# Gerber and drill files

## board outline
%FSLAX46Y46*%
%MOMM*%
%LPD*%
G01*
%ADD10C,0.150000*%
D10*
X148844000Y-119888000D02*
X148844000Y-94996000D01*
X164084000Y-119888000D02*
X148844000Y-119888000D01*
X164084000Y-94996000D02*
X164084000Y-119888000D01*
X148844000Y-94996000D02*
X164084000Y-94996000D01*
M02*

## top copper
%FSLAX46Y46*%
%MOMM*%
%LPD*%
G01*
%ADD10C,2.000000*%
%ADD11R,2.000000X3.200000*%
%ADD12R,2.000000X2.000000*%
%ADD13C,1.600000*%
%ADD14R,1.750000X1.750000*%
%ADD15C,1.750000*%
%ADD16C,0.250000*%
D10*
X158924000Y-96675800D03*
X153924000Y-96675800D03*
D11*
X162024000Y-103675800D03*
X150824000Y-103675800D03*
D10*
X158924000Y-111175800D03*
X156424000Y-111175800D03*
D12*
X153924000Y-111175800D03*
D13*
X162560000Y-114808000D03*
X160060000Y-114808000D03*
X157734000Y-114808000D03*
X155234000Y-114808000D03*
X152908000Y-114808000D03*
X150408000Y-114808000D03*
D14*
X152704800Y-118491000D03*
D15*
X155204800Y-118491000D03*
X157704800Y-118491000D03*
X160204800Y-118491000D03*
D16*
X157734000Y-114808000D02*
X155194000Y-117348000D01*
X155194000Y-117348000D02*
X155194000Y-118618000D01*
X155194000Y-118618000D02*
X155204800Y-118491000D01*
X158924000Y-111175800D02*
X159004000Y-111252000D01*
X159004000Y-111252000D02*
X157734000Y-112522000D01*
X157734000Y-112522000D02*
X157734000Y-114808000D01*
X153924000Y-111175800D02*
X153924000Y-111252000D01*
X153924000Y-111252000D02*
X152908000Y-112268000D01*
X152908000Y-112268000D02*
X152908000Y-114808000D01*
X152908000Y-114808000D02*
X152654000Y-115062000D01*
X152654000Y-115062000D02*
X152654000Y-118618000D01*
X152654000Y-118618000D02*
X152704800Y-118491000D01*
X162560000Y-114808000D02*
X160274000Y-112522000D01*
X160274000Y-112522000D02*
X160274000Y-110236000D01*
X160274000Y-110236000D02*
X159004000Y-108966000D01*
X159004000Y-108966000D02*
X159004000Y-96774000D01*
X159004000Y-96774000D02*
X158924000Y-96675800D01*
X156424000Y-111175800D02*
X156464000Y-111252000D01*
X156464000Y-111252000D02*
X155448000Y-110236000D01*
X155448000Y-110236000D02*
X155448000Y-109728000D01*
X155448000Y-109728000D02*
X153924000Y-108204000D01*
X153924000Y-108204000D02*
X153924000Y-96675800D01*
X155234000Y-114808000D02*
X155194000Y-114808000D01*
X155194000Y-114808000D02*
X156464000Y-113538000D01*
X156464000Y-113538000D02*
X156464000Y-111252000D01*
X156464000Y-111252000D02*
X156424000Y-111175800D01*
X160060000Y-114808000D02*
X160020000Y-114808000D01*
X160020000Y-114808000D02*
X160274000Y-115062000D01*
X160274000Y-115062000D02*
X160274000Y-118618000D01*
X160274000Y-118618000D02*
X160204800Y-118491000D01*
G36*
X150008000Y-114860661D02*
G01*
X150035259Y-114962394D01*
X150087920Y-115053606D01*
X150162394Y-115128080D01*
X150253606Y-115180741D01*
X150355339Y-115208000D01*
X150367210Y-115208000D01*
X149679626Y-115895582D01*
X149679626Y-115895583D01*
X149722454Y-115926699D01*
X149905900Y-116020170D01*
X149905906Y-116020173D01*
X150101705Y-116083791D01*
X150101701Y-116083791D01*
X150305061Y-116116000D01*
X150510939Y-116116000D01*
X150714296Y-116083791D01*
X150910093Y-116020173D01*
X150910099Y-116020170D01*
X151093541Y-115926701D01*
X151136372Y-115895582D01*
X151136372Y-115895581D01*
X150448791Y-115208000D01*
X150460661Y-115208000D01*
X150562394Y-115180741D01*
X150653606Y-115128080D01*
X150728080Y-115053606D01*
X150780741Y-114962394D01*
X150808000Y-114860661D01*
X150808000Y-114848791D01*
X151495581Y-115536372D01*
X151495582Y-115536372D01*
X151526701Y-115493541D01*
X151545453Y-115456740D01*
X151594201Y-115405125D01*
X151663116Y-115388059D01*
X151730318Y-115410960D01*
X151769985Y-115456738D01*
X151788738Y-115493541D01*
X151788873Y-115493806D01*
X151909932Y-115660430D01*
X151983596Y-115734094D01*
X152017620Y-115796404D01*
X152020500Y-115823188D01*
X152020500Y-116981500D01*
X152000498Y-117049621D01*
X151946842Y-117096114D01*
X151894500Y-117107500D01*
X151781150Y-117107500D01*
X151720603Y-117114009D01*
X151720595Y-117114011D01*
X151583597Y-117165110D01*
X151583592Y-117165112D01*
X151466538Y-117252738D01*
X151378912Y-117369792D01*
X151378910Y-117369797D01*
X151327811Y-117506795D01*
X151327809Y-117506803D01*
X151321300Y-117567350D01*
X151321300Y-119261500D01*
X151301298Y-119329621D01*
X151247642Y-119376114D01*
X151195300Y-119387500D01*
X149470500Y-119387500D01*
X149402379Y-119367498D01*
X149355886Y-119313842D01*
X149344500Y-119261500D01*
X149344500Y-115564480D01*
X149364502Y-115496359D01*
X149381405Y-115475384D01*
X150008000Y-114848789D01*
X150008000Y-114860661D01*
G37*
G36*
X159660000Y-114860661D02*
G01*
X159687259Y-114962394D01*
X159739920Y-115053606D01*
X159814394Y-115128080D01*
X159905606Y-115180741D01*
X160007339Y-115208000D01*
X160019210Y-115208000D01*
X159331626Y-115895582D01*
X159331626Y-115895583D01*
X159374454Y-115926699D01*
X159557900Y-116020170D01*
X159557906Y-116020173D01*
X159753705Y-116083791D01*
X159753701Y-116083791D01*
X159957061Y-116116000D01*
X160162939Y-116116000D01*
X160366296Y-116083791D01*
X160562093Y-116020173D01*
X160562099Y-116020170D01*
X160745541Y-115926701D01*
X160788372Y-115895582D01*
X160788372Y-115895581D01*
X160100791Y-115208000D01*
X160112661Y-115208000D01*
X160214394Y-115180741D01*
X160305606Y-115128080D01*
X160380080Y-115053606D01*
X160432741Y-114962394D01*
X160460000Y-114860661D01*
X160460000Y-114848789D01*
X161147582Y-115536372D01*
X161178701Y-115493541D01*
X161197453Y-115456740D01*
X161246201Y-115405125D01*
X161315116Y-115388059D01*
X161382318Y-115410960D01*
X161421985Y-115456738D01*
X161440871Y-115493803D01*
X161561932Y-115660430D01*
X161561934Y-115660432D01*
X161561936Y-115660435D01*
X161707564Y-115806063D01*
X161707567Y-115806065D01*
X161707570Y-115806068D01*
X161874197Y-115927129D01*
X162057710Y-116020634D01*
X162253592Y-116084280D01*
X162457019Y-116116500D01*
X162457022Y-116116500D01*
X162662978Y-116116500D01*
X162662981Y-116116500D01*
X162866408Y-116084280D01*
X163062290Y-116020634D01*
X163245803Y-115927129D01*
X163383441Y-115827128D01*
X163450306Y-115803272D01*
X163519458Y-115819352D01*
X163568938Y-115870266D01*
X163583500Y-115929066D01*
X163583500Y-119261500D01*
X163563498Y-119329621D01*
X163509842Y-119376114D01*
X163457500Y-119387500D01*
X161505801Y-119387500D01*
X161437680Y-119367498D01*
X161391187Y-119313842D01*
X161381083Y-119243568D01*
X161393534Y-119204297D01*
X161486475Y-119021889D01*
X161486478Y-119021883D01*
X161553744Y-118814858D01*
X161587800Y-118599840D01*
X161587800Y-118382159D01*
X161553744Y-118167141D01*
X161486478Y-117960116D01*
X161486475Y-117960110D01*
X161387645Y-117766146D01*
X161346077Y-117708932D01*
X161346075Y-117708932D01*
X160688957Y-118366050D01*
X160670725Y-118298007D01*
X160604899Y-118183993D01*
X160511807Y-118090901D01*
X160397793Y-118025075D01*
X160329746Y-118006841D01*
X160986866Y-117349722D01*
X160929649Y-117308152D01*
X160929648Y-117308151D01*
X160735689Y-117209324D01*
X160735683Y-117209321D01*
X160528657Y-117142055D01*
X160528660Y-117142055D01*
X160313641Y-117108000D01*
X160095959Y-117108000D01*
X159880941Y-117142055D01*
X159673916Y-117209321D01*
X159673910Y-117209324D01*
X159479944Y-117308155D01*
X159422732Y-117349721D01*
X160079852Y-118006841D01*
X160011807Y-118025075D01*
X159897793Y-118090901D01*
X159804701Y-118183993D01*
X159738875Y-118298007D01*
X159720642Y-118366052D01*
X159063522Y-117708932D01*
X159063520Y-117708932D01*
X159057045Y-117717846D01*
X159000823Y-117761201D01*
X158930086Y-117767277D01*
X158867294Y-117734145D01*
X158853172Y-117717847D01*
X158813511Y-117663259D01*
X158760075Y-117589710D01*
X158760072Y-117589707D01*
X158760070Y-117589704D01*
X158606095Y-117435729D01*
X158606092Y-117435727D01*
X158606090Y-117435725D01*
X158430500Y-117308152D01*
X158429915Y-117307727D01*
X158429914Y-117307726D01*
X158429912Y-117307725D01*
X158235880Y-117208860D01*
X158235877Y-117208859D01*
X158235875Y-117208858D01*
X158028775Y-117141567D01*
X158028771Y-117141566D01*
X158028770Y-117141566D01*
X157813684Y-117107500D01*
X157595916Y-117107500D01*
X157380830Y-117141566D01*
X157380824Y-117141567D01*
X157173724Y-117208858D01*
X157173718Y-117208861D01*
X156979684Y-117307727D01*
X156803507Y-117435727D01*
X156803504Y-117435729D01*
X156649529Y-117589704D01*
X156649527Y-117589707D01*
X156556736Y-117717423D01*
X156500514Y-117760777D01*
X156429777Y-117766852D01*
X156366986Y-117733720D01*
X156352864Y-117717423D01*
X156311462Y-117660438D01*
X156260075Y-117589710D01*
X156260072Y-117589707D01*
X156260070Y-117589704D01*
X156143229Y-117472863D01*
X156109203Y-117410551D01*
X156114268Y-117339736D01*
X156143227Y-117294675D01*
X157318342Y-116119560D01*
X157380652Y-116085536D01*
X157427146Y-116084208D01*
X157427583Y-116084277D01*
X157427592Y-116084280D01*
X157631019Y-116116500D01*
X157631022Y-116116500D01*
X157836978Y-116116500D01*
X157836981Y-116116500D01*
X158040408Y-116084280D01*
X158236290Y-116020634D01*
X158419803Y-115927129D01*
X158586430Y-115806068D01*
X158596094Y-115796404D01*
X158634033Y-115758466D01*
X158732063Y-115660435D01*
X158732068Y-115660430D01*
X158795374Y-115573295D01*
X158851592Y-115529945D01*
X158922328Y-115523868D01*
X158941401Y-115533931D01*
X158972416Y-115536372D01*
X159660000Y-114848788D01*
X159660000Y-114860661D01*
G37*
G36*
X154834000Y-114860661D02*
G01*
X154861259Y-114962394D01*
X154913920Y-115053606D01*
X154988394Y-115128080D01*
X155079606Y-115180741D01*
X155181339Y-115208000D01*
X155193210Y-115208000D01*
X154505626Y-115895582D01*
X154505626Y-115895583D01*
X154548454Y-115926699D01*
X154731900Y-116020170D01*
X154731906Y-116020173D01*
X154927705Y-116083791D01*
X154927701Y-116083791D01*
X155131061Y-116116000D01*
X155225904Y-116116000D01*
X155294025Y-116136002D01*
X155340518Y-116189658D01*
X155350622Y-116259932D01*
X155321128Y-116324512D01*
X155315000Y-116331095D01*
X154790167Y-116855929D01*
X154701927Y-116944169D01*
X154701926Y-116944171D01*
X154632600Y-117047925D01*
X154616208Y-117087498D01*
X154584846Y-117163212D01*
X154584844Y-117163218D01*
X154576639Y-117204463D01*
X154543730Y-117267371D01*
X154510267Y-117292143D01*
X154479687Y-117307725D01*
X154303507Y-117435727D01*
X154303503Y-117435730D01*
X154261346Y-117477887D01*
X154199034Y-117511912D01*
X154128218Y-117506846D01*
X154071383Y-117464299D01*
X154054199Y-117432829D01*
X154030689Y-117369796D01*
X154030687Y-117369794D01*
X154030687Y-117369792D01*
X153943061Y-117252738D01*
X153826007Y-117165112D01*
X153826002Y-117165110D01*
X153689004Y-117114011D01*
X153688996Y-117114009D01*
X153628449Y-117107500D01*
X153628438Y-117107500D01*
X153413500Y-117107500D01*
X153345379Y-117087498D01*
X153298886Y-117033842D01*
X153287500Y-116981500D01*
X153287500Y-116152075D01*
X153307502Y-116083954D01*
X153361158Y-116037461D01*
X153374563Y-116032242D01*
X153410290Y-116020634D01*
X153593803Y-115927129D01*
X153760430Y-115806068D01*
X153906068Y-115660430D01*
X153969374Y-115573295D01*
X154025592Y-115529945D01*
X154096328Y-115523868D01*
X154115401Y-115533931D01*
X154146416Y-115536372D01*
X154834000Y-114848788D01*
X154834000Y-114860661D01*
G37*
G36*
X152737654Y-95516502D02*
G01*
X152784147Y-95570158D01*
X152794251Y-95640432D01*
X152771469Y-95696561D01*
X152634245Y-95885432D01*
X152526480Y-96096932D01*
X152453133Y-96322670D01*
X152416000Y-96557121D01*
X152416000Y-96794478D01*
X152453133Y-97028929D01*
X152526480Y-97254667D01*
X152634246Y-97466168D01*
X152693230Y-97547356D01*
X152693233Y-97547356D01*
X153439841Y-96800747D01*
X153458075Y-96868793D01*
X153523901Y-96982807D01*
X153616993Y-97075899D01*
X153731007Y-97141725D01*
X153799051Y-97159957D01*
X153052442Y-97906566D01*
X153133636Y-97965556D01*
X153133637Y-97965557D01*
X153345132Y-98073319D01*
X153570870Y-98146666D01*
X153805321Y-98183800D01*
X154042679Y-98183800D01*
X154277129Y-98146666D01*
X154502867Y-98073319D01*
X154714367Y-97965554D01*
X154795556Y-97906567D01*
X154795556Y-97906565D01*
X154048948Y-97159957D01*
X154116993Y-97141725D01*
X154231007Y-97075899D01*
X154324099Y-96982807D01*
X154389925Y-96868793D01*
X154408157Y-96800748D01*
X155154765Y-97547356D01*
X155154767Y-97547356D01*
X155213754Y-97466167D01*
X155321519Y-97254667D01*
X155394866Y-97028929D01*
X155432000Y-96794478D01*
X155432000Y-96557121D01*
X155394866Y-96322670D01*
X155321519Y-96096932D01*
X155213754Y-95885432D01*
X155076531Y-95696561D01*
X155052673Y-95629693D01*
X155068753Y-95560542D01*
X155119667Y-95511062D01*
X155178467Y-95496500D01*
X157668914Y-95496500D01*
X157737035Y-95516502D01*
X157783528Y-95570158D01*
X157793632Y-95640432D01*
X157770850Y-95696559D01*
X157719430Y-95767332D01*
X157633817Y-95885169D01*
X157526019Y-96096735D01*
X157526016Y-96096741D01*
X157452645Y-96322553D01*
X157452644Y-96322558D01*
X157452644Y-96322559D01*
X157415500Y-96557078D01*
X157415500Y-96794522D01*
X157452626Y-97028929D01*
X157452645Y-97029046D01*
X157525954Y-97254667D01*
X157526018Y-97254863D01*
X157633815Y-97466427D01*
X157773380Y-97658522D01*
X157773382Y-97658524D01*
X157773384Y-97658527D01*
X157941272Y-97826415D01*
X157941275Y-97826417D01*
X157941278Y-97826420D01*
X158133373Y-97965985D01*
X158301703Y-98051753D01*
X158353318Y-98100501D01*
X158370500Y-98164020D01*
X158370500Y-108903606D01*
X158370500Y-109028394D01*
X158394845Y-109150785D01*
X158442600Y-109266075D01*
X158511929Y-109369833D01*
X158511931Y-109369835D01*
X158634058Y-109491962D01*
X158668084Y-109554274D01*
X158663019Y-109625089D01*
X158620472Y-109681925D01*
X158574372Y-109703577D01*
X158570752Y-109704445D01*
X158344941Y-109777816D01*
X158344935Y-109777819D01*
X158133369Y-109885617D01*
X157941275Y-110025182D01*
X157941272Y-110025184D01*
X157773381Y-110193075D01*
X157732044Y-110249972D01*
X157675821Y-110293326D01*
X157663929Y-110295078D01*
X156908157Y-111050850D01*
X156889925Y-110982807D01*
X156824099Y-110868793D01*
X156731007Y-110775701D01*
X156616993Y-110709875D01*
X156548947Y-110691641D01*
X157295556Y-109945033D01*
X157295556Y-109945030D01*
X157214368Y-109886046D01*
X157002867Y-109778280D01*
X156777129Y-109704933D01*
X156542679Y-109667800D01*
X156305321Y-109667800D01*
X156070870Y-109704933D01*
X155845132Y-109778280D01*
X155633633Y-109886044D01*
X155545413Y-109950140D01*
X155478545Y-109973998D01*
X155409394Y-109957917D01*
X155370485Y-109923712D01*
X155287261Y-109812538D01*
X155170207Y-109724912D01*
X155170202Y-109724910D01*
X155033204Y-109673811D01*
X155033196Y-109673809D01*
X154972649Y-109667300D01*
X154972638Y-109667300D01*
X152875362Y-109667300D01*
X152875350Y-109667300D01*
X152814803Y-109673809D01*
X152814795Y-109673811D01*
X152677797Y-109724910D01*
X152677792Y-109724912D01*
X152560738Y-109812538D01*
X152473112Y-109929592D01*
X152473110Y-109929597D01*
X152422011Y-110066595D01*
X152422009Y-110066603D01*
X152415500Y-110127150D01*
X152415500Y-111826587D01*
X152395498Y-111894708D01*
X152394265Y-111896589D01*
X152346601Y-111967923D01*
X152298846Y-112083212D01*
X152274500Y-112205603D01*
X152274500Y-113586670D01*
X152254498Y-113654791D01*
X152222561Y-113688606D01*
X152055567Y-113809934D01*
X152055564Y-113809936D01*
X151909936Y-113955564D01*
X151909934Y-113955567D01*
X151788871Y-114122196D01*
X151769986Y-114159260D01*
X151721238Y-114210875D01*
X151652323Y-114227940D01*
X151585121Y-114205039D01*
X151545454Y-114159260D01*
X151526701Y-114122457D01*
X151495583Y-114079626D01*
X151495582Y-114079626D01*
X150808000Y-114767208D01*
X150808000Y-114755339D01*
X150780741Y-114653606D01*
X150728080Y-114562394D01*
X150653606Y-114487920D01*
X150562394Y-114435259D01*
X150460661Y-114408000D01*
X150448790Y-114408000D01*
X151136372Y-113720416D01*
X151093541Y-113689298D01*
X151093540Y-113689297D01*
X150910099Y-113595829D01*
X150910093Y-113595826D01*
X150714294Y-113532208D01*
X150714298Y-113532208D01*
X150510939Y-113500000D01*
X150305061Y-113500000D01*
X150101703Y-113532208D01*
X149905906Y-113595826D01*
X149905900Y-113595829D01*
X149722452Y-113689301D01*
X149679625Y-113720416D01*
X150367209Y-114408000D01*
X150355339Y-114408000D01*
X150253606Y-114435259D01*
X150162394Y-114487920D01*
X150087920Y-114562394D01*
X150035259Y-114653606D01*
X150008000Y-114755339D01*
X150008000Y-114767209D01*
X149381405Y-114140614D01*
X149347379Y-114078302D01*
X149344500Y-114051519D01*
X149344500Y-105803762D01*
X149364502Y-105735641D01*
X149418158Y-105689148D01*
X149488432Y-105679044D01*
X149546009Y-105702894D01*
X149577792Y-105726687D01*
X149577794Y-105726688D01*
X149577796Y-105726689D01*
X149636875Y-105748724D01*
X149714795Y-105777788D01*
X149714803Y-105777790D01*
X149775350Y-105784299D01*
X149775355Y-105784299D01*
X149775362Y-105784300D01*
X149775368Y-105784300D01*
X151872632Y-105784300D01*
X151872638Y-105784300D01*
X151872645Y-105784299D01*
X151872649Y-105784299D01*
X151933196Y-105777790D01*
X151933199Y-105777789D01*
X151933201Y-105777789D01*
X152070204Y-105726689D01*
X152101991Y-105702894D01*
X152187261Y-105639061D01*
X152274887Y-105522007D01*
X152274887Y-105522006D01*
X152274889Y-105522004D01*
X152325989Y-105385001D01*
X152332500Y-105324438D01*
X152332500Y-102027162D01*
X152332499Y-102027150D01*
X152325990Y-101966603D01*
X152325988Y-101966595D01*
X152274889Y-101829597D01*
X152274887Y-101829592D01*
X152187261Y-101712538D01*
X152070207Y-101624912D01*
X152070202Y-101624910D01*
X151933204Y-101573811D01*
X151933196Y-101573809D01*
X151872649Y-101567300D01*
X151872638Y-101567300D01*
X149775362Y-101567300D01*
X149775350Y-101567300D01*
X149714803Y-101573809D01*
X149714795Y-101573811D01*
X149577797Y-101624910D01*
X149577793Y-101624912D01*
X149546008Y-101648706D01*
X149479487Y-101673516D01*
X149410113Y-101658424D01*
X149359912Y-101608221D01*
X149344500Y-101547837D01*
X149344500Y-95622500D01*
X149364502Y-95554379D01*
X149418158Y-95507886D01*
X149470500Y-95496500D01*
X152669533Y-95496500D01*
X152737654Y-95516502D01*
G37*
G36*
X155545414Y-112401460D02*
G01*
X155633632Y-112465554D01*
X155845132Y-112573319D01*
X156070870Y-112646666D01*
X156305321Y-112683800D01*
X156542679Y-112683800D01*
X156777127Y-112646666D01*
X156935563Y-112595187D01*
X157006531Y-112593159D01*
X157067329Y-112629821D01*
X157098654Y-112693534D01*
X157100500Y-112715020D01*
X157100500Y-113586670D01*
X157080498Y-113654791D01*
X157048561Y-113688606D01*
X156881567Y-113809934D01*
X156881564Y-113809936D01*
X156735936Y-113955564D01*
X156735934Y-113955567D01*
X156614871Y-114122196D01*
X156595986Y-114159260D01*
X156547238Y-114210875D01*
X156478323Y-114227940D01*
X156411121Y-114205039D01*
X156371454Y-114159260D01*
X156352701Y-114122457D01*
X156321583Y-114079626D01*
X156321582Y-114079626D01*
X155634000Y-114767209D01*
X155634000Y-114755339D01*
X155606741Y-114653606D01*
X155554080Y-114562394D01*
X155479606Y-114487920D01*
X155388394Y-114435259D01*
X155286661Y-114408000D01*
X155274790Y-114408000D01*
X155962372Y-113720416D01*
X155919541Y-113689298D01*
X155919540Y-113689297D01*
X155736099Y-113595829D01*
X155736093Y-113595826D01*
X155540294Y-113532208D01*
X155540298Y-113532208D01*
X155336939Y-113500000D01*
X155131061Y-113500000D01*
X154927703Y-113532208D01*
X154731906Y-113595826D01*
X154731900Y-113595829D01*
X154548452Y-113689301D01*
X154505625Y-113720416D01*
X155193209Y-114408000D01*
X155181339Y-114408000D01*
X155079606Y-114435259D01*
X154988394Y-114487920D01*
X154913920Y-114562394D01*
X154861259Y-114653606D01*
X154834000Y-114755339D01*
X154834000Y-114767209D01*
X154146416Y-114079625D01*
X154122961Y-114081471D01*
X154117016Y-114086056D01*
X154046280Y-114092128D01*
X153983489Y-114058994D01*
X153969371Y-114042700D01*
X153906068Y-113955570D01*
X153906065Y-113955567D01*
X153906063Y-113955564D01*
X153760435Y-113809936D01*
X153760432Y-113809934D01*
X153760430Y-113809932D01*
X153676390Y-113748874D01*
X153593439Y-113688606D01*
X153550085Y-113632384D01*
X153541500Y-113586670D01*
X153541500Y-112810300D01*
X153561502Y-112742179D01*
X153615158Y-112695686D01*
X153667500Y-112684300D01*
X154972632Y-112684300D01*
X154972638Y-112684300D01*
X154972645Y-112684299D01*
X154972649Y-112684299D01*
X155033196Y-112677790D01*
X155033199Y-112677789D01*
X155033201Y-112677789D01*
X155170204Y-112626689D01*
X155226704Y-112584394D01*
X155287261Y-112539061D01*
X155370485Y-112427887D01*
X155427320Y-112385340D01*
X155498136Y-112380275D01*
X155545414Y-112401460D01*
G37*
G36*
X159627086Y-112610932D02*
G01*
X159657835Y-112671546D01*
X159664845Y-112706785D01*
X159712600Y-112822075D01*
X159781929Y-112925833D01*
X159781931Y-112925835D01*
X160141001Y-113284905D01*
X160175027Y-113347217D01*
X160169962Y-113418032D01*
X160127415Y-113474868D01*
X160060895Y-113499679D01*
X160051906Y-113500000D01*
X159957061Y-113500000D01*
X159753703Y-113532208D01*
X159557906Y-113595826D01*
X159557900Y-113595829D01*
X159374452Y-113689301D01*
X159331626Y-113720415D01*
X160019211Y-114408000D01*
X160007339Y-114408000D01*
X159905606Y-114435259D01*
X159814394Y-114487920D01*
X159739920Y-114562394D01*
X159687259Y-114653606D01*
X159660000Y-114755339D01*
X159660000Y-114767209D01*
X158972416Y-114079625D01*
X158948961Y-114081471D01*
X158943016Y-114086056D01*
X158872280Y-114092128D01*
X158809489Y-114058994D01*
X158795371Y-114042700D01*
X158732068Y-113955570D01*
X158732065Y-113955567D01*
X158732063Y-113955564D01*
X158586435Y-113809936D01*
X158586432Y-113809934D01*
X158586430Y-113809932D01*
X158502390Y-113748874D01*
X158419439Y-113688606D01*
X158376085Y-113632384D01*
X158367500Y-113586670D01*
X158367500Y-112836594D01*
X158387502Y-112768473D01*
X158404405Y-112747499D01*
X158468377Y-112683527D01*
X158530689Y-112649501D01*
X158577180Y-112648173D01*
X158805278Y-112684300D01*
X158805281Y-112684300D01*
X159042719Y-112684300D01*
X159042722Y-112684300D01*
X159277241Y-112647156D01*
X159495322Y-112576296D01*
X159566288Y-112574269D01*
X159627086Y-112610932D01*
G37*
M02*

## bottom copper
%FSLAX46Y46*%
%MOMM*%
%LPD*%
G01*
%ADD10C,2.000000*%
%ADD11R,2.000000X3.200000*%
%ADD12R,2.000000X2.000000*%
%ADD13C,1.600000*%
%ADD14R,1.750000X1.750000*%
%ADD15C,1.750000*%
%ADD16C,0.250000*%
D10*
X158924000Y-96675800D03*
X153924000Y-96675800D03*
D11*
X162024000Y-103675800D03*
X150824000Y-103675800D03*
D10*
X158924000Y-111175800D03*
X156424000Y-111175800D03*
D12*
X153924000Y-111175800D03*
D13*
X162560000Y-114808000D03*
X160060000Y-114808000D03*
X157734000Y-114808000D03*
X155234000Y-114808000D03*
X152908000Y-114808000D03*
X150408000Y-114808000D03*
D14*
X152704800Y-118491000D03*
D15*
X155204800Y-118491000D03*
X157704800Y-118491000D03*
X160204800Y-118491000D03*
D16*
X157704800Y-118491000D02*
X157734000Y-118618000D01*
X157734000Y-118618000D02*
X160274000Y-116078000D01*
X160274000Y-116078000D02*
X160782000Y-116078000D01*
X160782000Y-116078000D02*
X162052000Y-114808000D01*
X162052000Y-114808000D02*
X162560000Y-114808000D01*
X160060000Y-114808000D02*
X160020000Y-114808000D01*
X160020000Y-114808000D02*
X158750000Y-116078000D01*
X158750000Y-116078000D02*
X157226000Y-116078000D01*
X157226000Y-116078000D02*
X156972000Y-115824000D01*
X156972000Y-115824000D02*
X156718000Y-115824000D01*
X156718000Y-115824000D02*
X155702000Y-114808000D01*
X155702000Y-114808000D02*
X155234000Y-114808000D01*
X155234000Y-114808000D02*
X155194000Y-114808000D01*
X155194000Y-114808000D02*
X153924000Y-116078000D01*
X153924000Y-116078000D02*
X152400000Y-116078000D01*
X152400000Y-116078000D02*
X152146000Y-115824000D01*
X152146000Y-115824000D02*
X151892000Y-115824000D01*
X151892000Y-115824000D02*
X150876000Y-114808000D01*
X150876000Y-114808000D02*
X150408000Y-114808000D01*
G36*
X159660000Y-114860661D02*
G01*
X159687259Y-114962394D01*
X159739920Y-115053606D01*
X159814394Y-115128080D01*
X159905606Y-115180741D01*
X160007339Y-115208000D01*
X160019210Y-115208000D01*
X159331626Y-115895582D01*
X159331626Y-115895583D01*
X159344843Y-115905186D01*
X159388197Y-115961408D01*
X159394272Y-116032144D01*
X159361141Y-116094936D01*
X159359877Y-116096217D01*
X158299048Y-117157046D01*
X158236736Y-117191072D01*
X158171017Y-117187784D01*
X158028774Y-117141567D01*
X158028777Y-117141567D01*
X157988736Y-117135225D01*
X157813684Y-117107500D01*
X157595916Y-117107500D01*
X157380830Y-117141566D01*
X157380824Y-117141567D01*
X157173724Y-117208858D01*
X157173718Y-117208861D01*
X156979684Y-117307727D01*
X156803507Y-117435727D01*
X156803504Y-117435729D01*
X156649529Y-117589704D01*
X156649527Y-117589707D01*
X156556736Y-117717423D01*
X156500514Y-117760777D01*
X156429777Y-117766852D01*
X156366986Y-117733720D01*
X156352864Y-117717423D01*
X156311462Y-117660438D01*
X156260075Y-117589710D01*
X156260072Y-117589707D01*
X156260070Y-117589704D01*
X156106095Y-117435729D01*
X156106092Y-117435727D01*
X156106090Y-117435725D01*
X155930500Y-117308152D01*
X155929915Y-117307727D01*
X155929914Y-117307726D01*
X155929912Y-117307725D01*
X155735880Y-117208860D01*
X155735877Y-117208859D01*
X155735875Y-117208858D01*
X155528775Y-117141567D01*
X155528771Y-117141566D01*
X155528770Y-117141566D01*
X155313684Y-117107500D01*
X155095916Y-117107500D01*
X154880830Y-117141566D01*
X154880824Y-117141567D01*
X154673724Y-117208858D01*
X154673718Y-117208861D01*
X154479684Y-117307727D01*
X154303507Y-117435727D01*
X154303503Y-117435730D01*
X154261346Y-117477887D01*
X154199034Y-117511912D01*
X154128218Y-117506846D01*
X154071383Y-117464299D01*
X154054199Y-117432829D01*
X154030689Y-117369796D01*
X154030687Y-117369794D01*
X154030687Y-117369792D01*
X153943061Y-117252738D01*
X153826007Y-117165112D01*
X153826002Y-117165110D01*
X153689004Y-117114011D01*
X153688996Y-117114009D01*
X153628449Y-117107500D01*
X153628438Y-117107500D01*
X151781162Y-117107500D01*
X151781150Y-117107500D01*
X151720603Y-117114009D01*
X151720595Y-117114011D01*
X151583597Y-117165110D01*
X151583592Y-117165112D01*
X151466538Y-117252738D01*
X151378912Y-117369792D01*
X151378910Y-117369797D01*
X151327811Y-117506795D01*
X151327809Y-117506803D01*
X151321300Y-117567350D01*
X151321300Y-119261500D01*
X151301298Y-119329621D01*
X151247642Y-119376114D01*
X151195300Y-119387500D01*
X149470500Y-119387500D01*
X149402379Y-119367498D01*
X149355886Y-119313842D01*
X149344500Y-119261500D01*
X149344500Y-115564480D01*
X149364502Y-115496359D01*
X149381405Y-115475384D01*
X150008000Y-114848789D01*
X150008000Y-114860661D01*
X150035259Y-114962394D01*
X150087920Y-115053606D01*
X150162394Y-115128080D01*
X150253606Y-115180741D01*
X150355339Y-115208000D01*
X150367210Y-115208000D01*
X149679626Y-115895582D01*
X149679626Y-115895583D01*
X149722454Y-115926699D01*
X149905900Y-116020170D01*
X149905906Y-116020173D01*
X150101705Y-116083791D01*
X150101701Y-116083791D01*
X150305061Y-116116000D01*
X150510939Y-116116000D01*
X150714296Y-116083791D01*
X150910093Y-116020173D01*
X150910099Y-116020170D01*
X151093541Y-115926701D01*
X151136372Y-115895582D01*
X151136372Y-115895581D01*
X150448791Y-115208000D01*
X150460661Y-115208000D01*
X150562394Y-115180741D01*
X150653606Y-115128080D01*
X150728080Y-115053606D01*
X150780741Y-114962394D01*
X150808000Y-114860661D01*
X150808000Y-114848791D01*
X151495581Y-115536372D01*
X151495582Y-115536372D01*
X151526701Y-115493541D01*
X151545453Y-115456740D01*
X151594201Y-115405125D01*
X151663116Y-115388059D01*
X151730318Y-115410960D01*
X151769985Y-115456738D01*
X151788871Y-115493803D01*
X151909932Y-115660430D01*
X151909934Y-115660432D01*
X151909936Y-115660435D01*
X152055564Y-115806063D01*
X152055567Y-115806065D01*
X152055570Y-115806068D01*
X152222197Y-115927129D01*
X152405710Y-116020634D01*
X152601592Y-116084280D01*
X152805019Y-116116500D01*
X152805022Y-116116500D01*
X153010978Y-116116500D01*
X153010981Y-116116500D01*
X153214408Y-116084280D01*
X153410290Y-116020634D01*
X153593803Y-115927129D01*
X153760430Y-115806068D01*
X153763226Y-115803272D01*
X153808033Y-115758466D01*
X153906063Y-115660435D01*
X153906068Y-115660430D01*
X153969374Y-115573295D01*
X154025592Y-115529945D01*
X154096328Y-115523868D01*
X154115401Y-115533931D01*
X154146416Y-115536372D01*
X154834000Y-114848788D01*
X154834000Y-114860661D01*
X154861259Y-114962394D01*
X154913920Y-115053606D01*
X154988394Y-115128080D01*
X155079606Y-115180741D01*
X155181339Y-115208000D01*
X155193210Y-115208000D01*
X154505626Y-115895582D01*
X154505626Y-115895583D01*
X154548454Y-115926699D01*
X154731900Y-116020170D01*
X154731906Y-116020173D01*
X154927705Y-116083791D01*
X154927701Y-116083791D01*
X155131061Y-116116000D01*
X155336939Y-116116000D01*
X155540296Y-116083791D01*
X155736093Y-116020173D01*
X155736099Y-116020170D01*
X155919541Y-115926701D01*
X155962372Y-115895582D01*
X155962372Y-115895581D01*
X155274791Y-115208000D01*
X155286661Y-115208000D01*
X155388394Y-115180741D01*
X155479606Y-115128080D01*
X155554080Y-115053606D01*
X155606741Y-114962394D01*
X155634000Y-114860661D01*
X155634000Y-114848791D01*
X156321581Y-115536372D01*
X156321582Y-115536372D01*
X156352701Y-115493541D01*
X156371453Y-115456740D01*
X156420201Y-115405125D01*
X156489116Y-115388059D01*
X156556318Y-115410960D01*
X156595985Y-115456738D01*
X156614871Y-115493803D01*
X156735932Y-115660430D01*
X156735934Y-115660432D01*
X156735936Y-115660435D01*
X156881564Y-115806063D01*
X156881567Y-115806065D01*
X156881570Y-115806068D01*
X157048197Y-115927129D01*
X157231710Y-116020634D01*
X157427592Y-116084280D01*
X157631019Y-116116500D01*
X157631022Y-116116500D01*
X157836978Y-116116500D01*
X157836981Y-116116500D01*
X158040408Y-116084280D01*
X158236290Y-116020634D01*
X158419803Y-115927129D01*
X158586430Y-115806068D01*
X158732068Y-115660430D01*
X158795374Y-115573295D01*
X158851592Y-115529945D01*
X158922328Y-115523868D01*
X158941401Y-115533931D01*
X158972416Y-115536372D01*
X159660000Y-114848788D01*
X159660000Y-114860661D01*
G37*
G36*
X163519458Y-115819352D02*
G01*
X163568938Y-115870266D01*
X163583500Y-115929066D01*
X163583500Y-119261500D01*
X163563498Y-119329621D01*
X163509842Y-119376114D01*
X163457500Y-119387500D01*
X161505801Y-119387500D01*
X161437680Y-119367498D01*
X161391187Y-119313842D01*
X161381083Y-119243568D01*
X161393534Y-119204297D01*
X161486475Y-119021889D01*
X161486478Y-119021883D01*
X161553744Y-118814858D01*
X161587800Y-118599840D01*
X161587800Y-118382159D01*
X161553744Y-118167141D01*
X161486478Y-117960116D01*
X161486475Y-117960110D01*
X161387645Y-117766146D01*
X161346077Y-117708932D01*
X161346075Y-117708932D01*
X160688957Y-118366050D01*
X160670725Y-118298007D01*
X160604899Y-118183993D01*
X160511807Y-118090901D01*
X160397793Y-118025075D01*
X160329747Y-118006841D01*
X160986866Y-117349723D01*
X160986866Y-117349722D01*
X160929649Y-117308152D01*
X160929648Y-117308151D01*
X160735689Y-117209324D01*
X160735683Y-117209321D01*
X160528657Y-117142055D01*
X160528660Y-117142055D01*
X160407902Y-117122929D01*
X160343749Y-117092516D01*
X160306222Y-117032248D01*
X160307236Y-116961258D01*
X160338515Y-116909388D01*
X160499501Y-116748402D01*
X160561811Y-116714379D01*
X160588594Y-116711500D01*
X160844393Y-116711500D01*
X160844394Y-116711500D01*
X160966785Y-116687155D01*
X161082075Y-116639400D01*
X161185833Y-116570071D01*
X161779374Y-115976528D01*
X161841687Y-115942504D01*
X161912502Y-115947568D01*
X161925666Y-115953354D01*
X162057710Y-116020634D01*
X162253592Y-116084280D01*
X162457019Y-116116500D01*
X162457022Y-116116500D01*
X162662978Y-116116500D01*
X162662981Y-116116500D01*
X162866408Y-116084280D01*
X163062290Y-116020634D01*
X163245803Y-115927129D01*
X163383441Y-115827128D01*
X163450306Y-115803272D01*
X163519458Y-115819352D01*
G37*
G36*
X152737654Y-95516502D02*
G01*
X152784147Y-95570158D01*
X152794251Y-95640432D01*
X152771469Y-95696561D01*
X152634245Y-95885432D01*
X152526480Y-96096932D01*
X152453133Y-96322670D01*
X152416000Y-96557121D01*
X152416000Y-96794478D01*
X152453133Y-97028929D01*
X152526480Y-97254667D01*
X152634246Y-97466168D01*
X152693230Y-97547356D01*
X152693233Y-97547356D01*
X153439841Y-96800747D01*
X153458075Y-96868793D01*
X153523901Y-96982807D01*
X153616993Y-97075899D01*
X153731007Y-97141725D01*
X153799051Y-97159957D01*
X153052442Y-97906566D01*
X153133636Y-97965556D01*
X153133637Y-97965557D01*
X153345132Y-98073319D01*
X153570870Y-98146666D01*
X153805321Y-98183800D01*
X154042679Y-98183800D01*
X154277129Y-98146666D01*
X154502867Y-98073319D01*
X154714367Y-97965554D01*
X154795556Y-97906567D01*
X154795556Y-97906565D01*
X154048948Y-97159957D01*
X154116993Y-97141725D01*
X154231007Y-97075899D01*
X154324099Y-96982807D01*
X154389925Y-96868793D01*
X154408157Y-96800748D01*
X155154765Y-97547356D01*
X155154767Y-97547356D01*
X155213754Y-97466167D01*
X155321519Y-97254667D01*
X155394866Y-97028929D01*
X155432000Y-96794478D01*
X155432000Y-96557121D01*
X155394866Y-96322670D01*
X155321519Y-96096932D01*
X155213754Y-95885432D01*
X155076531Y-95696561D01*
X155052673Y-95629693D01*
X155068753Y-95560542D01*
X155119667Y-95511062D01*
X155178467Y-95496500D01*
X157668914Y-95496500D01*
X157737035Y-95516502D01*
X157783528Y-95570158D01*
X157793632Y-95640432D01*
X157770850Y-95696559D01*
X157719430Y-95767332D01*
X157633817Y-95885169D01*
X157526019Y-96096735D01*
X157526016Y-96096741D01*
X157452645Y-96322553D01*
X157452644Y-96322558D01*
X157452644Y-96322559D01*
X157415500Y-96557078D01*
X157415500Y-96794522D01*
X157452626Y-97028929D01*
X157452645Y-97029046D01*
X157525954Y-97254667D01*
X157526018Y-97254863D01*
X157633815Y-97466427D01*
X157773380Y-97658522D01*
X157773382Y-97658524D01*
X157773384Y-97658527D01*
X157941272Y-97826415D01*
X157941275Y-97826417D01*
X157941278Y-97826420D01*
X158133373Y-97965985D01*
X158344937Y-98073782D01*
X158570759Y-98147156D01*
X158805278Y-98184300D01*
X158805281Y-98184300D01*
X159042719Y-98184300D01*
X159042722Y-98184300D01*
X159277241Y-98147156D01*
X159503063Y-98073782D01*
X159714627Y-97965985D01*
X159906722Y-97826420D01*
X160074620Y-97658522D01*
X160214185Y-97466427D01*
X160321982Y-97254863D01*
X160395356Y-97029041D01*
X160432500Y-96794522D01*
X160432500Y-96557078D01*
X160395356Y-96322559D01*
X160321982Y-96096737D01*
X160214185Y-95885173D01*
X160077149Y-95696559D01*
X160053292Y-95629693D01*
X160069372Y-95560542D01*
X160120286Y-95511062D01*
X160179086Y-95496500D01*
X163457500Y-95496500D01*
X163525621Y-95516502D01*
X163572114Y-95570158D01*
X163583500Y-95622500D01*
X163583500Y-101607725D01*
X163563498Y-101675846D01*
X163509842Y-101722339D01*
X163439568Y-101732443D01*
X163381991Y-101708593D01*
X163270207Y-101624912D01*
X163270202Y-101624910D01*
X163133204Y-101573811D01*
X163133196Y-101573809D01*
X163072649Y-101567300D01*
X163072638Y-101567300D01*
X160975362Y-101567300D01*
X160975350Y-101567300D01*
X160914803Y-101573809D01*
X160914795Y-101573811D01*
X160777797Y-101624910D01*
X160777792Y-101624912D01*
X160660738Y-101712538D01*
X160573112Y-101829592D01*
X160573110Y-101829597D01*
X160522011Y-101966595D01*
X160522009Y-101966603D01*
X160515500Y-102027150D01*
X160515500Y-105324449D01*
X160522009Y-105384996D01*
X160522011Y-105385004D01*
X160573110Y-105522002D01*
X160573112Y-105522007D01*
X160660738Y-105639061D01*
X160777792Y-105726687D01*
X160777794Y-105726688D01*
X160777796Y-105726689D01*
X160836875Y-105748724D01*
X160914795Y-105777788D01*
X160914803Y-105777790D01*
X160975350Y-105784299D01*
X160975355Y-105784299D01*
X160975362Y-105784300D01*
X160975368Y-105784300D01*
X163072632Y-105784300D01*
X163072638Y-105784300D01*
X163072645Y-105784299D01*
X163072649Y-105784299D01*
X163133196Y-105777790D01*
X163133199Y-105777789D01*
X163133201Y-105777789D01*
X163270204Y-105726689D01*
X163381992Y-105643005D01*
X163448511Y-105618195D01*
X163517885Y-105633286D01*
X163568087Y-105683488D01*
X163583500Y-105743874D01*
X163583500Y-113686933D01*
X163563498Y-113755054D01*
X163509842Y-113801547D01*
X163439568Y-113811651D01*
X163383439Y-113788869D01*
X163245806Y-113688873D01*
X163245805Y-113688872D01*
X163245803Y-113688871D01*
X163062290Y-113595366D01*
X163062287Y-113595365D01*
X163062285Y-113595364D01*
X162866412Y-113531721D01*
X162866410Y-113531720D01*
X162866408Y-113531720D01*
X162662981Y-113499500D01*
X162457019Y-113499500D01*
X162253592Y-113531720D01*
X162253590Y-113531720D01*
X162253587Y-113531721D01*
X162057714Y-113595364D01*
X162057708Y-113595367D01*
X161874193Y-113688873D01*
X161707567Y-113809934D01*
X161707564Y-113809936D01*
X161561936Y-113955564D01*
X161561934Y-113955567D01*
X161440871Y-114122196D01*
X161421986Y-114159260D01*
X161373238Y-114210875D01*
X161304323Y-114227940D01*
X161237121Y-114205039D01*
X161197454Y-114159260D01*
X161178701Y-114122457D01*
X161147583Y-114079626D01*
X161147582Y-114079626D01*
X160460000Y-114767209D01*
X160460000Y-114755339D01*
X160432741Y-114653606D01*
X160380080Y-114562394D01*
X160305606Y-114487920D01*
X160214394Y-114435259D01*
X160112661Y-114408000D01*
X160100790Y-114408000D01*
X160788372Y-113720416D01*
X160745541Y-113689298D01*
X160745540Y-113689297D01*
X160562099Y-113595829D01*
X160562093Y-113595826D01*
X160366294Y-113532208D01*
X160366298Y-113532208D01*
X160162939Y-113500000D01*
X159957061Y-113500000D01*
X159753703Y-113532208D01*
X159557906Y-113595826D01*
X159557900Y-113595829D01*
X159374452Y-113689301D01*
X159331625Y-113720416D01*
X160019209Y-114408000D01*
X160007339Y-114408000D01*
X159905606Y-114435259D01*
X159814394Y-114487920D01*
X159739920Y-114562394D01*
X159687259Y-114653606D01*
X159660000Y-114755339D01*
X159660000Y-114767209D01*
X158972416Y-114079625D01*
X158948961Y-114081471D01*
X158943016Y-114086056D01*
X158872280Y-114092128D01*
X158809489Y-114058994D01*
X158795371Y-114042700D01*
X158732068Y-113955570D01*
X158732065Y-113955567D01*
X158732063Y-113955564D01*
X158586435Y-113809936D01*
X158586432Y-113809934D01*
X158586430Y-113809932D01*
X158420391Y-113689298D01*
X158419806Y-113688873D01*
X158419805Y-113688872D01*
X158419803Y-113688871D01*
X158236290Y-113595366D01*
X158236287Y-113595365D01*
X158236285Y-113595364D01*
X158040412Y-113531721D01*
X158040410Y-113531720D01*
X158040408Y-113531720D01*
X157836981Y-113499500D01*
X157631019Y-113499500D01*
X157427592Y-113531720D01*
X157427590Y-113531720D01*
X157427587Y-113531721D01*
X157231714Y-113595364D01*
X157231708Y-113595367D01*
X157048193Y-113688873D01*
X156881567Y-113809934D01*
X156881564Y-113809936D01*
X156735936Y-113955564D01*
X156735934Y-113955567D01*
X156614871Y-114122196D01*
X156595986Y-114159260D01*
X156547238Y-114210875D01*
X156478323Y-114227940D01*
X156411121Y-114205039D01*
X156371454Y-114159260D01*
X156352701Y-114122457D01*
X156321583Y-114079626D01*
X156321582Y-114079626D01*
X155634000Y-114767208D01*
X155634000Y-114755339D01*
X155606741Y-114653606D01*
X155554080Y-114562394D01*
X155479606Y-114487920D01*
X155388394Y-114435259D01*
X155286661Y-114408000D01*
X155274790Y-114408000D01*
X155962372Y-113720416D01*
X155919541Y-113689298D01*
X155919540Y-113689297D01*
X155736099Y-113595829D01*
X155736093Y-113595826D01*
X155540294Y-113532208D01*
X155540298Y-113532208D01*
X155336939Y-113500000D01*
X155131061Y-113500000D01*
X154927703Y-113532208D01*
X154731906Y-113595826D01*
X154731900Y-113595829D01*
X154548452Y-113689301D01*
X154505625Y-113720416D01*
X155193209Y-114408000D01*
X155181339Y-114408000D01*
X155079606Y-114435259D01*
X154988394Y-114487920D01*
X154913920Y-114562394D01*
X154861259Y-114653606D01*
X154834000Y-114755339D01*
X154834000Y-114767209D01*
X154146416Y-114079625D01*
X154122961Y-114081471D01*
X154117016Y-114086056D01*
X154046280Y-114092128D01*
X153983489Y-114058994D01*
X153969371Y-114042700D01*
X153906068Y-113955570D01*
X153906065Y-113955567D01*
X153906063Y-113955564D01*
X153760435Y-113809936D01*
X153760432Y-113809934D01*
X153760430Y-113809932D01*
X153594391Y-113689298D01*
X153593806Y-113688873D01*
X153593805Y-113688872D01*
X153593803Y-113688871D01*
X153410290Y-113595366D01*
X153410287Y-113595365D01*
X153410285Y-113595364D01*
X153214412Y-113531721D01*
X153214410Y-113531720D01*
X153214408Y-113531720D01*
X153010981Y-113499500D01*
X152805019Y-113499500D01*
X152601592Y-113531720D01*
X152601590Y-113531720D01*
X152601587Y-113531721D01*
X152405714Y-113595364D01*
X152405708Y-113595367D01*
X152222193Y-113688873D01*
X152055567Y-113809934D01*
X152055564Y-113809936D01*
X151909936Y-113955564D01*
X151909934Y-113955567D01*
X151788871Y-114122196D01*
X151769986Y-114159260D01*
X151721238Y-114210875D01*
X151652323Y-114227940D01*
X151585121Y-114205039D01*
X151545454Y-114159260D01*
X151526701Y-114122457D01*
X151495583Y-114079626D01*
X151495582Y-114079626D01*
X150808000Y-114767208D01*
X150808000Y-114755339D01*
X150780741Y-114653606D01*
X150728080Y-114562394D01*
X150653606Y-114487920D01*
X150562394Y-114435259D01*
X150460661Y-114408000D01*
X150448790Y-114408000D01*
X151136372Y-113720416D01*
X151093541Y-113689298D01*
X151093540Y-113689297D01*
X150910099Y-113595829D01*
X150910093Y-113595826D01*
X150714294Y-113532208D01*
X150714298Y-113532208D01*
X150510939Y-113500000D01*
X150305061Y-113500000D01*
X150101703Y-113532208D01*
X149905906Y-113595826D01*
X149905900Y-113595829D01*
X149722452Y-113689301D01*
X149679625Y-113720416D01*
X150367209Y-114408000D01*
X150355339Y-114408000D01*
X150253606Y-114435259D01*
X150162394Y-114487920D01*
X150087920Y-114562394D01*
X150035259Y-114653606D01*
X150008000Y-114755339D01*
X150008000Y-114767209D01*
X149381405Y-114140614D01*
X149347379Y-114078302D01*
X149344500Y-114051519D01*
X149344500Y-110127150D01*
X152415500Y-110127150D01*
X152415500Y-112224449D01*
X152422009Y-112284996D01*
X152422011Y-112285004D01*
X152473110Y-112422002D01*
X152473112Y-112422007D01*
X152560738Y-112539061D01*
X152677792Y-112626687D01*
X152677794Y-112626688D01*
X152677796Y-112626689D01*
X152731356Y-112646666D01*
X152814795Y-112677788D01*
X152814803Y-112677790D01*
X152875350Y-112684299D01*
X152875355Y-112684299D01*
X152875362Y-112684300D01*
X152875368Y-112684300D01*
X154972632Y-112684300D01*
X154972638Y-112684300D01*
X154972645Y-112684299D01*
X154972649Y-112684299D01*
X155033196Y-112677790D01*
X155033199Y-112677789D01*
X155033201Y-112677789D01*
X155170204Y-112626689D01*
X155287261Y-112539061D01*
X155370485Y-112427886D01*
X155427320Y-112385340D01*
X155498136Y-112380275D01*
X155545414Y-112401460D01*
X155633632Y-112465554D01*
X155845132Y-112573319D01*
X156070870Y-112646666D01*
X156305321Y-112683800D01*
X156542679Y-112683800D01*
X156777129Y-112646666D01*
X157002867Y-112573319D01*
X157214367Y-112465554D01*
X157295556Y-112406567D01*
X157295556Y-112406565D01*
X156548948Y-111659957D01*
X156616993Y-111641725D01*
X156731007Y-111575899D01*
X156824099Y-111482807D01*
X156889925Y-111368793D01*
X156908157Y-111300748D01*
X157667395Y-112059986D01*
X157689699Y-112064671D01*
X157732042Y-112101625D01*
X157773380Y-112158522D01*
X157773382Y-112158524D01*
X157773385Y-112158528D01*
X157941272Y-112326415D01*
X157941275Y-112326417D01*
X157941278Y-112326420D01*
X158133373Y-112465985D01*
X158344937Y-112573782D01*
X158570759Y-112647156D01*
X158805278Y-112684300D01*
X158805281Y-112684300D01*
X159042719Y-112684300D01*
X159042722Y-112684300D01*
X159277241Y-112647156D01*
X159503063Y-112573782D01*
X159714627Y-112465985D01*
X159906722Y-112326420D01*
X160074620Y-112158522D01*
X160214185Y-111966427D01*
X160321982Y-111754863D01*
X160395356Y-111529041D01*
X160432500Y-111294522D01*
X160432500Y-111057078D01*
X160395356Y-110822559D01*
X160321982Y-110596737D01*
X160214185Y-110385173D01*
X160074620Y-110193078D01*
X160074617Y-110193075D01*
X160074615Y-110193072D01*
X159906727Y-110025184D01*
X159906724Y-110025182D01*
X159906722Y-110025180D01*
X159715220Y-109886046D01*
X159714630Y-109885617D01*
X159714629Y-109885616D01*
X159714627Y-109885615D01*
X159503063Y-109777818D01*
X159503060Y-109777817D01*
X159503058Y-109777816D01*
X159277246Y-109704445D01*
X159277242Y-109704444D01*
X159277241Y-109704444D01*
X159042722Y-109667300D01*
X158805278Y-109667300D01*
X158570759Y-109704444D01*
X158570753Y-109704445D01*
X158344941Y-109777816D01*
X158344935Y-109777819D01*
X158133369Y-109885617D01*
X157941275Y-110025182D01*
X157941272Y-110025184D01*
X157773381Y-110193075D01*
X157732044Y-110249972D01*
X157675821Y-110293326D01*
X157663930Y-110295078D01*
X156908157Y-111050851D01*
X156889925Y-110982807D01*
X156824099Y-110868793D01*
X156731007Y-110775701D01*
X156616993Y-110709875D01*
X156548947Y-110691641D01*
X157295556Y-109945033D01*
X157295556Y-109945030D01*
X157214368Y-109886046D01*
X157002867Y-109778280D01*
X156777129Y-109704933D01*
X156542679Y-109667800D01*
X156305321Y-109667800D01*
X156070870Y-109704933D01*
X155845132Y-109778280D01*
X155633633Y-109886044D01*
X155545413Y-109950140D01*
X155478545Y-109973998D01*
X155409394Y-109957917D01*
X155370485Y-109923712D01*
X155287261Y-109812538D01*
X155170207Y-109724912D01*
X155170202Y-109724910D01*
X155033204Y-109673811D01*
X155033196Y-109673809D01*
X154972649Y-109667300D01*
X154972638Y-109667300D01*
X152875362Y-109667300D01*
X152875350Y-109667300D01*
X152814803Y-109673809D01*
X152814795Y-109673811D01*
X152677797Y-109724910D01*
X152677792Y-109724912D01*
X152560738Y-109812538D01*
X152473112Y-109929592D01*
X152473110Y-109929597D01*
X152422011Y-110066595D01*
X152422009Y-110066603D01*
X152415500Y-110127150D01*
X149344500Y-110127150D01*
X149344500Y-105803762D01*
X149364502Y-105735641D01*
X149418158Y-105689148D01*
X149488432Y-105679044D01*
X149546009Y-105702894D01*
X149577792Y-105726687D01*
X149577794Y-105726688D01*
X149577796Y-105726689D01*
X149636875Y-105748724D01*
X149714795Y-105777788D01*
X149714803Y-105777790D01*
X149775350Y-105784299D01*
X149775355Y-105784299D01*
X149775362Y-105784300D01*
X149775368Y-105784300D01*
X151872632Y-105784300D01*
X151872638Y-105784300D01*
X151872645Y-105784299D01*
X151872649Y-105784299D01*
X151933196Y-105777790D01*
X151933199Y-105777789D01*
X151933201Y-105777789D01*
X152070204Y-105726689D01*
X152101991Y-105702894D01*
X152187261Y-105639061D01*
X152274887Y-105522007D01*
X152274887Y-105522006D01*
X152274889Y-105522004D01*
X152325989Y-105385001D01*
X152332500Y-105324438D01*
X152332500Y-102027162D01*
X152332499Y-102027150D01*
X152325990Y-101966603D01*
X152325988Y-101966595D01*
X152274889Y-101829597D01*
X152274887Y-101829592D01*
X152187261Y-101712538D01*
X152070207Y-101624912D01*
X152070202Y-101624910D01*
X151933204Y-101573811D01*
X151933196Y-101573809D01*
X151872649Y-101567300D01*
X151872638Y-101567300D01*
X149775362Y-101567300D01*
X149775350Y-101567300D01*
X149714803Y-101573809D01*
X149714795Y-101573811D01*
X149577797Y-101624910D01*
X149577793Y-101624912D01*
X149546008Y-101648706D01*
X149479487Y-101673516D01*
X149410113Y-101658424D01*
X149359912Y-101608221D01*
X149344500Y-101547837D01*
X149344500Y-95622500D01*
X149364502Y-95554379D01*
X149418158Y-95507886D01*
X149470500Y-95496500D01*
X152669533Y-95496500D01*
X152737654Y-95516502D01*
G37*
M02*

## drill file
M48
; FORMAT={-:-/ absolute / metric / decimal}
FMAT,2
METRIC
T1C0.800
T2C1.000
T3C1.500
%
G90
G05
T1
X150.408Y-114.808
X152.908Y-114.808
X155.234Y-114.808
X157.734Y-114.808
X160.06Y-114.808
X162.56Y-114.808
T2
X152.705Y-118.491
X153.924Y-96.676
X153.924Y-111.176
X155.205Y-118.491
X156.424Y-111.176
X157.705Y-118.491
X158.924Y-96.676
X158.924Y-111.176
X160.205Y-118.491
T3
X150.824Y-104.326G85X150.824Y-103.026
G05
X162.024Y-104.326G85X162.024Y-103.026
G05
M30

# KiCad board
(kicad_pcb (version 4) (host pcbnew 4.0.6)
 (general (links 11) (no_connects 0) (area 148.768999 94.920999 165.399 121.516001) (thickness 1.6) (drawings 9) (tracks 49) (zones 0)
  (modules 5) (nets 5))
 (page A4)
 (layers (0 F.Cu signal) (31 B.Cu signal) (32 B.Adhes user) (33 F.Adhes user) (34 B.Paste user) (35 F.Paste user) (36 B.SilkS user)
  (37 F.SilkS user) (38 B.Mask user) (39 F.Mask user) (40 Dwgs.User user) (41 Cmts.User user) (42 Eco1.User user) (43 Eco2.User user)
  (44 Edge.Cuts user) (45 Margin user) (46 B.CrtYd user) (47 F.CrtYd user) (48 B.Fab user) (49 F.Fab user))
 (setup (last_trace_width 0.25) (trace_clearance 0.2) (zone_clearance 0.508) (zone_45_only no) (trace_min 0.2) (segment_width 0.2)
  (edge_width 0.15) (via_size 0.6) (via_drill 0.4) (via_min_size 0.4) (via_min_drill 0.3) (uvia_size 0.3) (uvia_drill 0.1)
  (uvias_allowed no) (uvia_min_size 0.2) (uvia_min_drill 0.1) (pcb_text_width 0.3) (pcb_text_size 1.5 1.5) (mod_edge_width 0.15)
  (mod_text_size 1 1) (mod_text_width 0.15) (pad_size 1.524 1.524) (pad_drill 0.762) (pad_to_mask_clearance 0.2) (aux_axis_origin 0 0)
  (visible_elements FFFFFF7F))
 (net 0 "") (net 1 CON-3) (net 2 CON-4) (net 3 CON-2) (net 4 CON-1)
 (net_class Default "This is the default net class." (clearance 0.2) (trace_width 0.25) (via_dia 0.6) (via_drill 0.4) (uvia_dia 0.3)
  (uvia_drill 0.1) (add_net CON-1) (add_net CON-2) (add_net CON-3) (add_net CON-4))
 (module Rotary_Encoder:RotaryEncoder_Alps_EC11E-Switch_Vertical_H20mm (layer F.Cu) (at 153.924 111.1758 90)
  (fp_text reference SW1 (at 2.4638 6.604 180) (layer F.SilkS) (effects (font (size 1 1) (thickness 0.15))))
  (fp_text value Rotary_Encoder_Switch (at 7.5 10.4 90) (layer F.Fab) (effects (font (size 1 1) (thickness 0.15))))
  (pad 4 thru_hole circle (at 14.5 5 90) (size 2 2) (drill 1) (layers *.Cu *.Mask) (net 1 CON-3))
  (pad 5 thru_hole circle (at 14.5 0 90) (size 2 2) (drill 1) (layers *.Cu *.Mask) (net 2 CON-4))
  (pad MP thru_hole rect (at 7.5 8.1 90) (size 3.2 2) (drill oval 2.8 1.5) (layers *.Cu *.Mask))
  (pad MP thru_hole rect (at 7.5 -3.1 90) (size 3.2 2) (drill oval 2.8 1.5) (layers *.Cu *.Mask))
  (pad 3 thru_hole circle (at 0 5 90) (size 2 2) (drill 1) (layers *.Cu *.Mask) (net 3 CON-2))
  (pad 2 thru_hole circle (at 0 2.5 90) (size 2 2) (drill 1) (layers *.Cu *.Mask) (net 2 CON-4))
  (pad 1 thru_hole rect (at 0 0 90) (size 2 2) (drill 1) (layers *.Cu *.Mask) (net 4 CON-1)))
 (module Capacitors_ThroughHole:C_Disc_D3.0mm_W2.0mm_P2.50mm (layer F.Cu) (at 162.56 114.808 180)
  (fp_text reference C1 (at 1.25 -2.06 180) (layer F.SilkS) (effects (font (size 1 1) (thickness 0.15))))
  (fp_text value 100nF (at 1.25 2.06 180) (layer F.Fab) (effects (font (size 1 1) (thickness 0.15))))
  (pad 1 thru_hole circle (at 0 0 180) (size 1.6 1.6) (drill 0.8) (layers *.Cu *.Mask) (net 1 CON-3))
  (pad 2 thru_hole circle (at 2.5 0 180) (size 1.6 1.6) (drill 0.8) (layers *.Cu *.Mask) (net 2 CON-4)))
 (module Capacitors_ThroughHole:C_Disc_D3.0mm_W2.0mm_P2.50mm (layer F.Cu) (at 157.734 114.808 180)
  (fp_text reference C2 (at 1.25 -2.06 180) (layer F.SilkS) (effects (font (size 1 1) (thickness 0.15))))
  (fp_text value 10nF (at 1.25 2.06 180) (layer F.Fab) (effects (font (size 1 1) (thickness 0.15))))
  (pad 1 thru_hole circle (at 0 0 180) (size 1.6 1.6) (drill 0.8) (layers *.Cu *.Mask) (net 3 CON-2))
  (pad 2 thru_hole circle (at 2.5 0 180) (size 1.6 1.6) (drill 0.8) (layers *.Cu *.Mask) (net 2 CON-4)))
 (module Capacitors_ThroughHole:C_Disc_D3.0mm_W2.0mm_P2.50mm (layer F.Cu) (at 152.908 114.808 180)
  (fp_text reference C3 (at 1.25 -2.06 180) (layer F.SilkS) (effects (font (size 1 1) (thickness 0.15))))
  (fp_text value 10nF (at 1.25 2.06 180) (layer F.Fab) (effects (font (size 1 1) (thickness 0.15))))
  (pad 1 thru_hole circle (at 0 0 180) (size 1.6 1.6) (drill 0.8) (layers *.Cu *.Mask) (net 4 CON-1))
  (pad 2 thru_hole circle (at 2.5 0 180) (size 1.6 1.6) (drill 0.8) (layers *.Cu *.Mask) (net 2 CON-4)))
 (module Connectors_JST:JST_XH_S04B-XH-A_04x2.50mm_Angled (layer B.Cu) (at 152.7048 118.491)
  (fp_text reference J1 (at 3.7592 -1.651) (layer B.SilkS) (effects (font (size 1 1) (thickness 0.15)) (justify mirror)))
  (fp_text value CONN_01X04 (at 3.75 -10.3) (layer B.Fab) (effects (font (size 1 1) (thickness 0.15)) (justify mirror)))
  (pad 1 thru_hole rect (at 0 0) (size 1.75 1.75) (drill 1) (layers *.Cu *.Mask B.SilkS) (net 4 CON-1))
  (pad 2 thru_hole circle (at 2.5 0) (size 1.75 1.75) (drill 1) (layers *.Cu *.Mask B.SilkS) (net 3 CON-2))
  (pad 3 thru_hole circle (at 5 0) (size 1.75 1.75) (drill 1) (layers *.Cu *.Mask B.SilkS) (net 1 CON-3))
  (pad 4 thru_hole circle (at 7.5 0) (size 1.75 1.75) (drill 1) (layers *.Cu *.Mask B.SilkS) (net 2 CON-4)))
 (gr_line (start 148.844 119.888) (end 148.844 94.996) (angle 90) (layer Edge.Cuts) (width 0.15))
 (gr_line (start 164.084 119.888) (end 148.844 119.888) (angle 90) (layer Edge.Cuts) (width 0.15))
 (gr_line (start 164.084 94.996) (end 164.084 119.888) (angle 90) (layer Edge.Cuts) (width 0.15))
 (gr_line (start 148.844 94.996) (end 164.084 94.996) (angle 90) (layer Edge.Cuts) (width 0.15))
 (segment (start 157.734 114.808) (end 155.194 117.348) (width 0.25) (layer F.Cu) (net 3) (status 80000))
 (segment (start 155.194 117.348) (end 155.194 118.618) (width 0.25) (layer F.Cu) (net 3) (status 80000))
 (segment (start 155.194 118.618) (end 155.2048 118.491) (width 0.25) (layer F.Cu) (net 3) (status 80000))
 (segment (start 158.924 111.1758) (end 159.004 111.252) (width 0.25) (layer F.Cu) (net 3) (status 80000))
 (segment (start 159.004 111.252) (end 157.734 112.522) (width 0.25) (layer F.Cu) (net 3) (status 80000))
 (segment (start 157.734 112.522) (end 157.734 114.808) (width 0.25) (layer F.Cu) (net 3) (status 80000))
 (segment (start 153.924 111.1758) (end 153.924 111.252) (width 0.25) (layer F.Cu) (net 4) (status 80000))
 (segment (start 153.924 111.252) (end 152.908 112.268) (width 0.25) (layer F.Cu) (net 4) (status 80000))
 (segment (start 152.908 112.268) (end 152.908 114.808) (width 0.25) (layer F.Cu) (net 4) (status 80000))
 (segment (start 152.908 114.808) (end 152.654 115.062) (width 0.25) (layer F.Cu) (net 4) (status 80000))
 (segment (start 152.654 115.062) (end 152.654 118.618) (width 0.25) (layer F.Cu) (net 4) (status 80000))
 (segment (start 152.654 118.618) (end 152.7048 118.491) (width 0.25) (layer F.Cu) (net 4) (status 80000))
 (segment (start 162.56 114.808) (end 160.274 112.522) (width 0.25) (layer F.Cu) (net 1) (status 80000))
 (segment (start 160.274 112.522) (end 160.274 110.236) (width 0.25) (layer F.Cu) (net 1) (status 80000))
 (segment (start 160.274 110.236) (end 159.004 108.966) (width 0.25) (layer F.Cu) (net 1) (status 80000))
 (segment (start 159.004 108.966) (end 159.004 96.774) (width 0.25) (layer F.Cu) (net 1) (status 80000))
 (segment (start 159.004 96.774) (end 158.924 96.6758) (width 0.25) (layer F.Cu) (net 1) (status 80000))
 (segment (start 157.7048 118.491) (end 157.734 118.618) (width 0.25) (layer B.Cu) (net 1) (status 80000))
 (segment (start 157.734 118.618) (end 160.274 116.078) (width 0.25) (layer B.Cu) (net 1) (status 80000))
 (segment (start 160.274 116.078) (end 160.782 116.078) (width 0.25) (layer B.Cu) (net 1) (status 80000))
 (segment (start 160.782 116.078) (end 162.052 114.808) (width 0.25) (layer B.Cu) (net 1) (status 80000))
 (segment (start 162.052 114.808) (end 162.56 114.808) (width 0.25) (layer B.Cu) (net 1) (status 80000))
 (segment (start 156.424 111.1758) (end 156.464 111.252) (width 0.25) (layer F.Cu) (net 2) (status 80000))
 (segment (start 156.464 111.252) (end 155.448 110.236) (width 0.25) (layer F.Cu) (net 2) (status 80000))
 (segment (start 155.448 110.236) (end 155.448 109.728) (width 0.25) (layer F.Cu) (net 2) (status 80000))
 (segment (start 155.448 109.728) (end 153.924 108.204) (width 0.25) (layer F.Cu) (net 2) (status 80000))
 (segment (start 153.924 108.204) (end 153.924 96.6758) (width 0.25) (layer F.Cu) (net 2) (status 80000))
 (segment (start 155.234 114.808) (end 155.194 114.808) (width 0.25) (layer F.Cu) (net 2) (status 80000))
 (segment (start 155.194 114.808) (end 156.464 113.538) (width 0.25) (layer F.Cu) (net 2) (status 80000))
 (segment (start 156.464 113.538) (end 156.464 111.252) (width 0.25) (layer F.Cu) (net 2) (status 80000))
 (segment (start 156.464 111.252) (end 156.424 111.1758) (width 0.25) (layer F.Cu) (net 2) (status 80000))
 (segment (start 160.06 114.808) (end 160.02 114.808) (width 0.25) (layer B.Cu) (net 2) (status 80000))
 (segment (start 160.02 114.808) (end 158.75 116.078) (width 0.25) (layer B.Cu) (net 2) (status 80000))
 (segment (start 158.75 116.078) (end 157.226 116.078) (width 0.25) (layer B.Cu) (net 2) (status 80000))
 (segment (start 157.226 116.078) (end 156.972 115.824) (width 0.25) (layer B.Cu) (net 2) (status 80000))
 (segment (start 156.972 115.824) (end 156.718 115.824) (width 0.25) (layer B.Cu) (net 2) (status 80000))
 (segment (start 156.718 115.824) (end 155.702 114.808) (width 0.25) (layer B.Cu) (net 2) (status 80000))
 (segment (start 155.702 114.808) (end 155.234 114.808) (width 0.25) (layer B.Cu) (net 2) (status 80000))
 (segment (start 155.234 114.808) (end 155.194 114.808) (width 0.25) (layer B.Cu) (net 2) (status 80000))
 (segment (start 155.194 114.808) (end 153.924 116.078) (width 0.25) (layer B.Cu) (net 2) (status 80000))
 (segment (start 153.924 116.078) (end 152.4 116.078) (width 0.25) (layer B.Cu) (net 2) (status 80000))
 (segment (start 152.4 116.078) (end 152.146 115.824) (width 0.25) (layer B.Cu) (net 2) (status 80000))
 (segment (start 152.146 115.824) (end 151.892 115.824) (width 0.25) (layer B.Cu) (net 2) (status 80000))
 (segment (start 151.892 115.824) (end 150.876 114.808) (width 0.25) (layer B.Cu) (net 2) (status 80000))
 (segment (start 150.876 114.808) (end 150.408 114.808) (width 0.25) (layer B.Cu) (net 2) (status 80000))
 (segment (start 160.06 114.808) (end 160.02 114.808) (width 0.25) (layer F.Cu) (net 2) (status 80000))
 (segment (start 160.02 114.808) (end 160.274 115.062) (width 0.25) (layer F.Cu) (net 2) (status 80000))
 (segment (start 160.274 115.062) (end 160.274 118.618) (width 0.25) (layer F.Cu) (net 2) (status 80000))
 (segment (start 160.274 118.618) (end 160.2048 118.491) (width 0.25) (layer F.Cu) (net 2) (status 80000))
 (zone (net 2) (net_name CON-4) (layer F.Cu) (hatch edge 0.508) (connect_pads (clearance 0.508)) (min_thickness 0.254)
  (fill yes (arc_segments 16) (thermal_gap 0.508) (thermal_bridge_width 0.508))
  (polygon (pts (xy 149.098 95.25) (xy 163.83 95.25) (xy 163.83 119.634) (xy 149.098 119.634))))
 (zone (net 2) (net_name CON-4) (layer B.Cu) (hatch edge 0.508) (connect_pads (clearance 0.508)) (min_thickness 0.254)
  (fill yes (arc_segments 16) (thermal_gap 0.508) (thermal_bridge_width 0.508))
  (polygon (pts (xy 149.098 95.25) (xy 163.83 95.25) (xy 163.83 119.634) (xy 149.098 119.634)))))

